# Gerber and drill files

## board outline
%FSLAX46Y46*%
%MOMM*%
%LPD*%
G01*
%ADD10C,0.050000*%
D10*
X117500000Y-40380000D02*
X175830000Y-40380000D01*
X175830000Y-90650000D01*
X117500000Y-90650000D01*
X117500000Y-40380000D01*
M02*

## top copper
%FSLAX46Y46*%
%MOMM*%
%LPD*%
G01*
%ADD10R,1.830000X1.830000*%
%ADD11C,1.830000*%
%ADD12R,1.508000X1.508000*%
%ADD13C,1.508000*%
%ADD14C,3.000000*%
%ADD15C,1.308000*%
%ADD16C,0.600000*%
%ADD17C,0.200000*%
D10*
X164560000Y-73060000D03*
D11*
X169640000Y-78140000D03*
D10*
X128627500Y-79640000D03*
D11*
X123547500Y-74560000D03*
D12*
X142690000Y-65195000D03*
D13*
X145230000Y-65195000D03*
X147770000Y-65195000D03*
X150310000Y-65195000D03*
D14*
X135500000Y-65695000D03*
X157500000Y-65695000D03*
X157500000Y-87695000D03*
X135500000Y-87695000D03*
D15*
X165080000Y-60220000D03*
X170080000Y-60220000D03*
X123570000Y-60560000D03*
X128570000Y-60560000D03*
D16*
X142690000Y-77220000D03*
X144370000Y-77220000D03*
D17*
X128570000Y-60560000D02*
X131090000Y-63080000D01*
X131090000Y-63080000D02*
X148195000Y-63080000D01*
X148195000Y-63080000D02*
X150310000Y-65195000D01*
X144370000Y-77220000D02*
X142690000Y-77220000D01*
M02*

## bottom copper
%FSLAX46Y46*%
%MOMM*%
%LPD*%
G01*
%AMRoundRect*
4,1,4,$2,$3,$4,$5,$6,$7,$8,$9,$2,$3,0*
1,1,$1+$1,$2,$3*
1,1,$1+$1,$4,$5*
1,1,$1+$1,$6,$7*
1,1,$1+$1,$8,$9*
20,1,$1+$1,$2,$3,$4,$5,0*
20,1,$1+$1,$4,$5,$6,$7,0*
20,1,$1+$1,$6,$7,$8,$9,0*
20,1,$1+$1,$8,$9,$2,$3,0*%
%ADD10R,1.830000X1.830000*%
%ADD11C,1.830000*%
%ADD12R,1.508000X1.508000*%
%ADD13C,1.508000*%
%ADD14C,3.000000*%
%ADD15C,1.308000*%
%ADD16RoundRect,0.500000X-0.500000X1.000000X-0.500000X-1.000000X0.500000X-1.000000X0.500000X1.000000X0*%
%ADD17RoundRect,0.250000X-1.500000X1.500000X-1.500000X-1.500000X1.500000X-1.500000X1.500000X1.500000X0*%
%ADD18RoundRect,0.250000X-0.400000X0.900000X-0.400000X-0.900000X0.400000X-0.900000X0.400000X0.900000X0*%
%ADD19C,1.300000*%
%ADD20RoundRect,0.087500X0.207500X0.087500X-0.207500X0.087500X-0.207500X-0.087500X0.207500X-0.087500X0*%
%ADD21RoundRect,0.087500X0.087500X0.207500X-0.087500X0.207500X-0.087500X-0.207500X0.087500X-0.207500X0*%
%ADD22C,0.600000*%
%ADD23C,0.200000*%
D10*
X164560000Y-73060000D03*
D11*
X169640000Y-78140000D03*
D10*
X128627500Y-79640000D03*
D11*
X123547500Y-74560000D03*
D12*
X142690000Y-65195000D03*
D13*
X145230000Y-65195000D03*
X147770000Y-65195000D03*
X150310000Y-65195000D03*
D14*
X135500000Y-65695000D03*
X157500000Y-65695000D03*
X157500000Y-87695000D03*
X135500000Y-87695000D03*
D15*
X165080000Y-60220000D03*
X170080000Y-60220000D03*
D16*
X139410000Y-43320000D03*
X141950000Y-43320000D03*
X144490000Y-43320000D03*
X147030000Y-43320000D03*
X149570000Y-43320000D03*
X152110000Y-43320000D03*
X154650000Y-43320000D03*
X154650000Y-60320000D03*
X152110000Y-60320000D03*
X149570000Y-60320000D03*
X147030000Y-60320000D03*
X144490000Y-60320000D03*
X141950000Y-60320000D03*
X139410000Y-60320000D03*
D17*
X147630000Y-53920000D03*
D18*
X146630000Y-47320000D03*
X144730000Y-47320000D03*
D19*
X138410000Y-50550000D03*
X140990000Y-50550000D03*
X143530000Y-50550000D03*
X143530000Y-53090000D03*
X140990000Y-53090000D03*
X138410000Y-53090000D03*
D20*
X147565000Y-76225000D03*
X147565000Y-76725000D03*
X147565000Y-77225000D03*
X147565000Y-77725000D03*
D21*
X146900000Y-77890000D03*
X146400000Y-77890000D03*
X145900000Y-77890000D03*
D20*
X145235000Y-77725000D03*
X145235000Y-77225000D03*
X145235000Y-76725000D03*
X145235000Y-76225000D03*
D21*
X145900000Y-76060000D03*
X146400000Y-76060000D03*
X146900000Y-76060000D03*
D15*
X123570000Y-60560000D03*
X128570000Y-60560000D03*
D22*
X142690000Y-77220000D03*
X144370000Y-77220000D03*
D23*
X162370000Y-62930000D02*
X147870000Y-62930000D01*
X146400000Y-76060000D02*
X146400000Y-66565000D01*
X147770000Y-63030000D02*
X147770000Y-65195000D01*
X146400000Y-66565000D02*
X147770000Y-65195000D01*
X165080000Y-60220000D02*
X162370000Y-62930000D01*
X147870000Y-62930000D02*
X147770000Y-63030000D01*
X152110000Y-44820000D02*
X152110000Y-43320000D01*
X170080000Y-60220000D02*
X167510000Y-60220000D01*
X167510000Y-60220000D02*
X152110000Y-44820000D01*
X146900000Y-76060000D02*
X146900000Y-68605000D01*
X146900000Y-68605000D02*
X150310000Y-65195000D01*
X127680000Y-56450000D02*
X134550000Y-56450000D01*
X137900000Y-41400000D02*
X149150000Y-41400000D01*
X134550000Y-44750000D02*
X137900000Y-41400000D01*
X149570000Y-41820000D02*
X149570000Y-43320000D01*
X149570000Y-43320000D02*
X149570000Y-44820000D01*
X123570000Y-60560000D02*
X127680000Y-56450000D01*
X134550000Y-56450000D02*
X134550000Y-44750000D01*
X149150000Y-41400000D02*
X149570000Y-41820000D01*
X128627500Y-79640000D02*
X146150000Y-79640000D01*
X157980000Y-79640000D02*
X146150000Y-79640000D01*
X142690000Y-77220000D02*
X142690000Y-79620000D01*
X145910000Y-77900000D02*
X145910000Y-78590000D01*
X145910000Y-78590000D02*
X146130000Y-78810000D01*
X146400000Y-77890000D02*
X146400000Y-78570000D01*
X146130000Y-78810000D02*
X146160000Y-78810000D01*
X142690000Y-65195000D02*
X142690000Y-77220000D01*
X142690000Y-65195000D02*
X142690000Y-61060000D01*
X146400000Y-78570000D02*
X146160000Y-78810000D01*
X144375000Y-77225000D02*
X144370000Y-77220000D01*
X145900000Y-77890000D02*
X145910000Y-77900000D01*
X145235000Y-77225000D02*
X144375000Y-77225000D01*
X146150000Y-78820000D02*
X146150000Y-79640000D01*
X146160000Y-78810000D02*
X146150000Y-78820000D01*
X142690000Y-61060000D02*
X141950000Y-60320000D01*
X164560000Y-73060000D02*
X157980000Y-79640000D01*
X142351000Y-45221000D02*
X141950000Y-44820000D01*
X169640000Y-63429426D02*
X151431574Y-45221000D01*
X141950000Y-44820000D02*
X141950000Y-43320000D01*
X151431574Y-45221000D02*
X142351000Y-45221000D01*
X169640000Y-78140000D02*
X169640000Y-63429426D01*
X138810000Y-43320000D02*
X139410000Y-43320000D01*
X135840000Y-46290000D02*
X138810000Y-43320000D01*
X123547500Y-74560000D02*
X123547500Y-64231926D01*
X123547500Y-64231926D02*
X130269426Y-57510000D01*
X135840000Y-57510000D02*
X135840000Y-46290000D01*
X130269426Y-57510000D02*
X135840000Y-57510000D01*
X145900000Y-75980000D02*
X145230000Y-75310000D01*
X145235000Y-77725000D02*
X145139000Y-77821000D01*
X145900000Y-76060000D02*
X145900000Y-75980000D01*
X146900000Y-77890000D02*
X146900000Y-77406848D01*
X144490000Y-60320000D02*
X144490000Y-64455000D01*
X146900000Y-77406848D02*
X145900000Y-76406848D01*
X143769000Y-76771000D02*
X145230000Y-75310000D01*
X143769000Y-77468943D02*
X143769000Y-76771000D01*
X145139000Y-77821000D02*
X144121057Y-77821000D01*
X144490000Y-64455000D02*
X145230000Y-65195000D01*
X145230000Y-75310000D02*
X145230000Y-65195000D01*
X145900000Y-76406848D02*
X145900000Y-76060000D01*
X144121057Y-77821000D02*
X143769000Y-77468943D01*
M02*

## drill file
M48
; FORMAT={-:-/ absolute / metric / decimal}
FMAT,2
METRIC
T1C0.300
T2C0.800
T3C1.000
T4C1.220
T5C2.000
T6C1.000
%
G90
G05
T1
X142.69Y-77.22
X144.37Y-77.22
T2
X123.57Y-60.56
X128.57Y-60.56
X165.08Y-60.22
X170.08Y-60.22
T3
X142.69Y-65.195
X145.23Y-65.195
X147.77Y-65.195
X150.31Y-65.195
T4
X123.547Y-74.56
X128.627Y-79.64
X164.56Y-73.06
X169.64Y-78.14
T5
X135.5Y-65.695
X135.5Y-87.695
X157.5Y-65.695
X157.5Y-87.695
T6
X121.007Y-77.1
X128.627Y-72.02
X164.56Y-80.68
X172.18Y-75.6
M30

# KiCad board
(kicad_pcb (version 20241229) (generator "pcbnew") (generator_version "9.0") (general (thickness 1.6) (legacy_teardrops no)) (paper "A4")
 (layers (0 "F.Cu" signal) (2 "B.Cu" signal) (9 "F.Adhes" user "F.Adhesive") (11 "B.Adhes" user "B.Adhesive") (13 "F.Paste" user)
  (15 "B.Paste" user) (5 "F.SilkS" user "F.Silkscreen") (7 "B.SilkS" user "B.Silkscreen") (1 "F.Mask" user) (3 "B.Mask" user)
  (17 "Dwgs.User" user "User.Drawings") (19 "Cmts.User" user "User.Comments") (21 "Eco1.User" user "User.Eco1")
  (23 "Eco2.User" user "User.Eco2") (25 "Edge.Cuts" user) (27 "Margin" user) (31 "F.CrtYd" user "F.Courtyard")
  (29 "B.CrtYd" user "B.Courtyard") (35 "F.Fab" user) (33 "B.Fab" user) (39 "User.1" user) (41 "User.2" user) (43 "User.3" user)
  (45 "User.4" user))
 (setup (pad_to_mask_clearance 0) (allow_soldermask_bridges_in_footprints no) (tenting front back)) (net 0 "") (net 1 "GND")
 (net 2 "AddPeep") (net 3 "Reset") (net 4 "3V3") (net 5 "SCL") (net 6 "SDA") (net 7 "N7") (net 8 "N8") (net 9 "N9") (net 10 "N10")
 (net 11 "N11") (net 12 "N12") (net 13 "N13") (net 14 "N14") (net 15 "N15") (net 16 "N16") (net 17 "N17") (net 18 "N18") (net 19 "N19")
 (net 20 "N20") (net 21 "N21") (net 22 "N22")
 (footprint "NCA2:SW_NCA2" (layer "F.Cu") (at 168.37 76.87 180)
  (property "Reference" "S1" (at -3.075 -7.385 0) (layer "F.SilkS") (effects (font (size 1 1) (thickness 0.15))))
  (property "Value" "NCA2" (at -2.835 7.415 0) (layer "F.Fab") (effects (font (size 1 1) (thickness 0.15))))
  (pad "" np_thru_hole circle (at -3.81 1.27 180) (size 1 1) (drill 1) (layers "*.Cu" "*.Mask"))
  (pad "" np_thru_hole circle (at 3.81 -3.81 180) (size 1 1) (drill 1) (layers "*.Cu" "*.Mask"))
  (pad "1" thru_hole rect (at 3.81 3.81 180) (size 1.83 1.83) (drill 1.22) (layers "*.Cu" "*.Mask") (remove_unused_layers no) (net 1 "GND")
   (solder_mask_margin 0.102))
  (pad "3" thru_hole circle (at -1.27 -1.27 180) (size 1.83 1.83) (drill 1.22) (layers "*.Cu" "*.Mask") (remove_unused_layers no)
   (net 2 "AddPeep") (solder_mask_margin 0.102)))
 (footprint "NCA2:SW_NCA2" (layer "F.Cu") (at 124.8175 75.83)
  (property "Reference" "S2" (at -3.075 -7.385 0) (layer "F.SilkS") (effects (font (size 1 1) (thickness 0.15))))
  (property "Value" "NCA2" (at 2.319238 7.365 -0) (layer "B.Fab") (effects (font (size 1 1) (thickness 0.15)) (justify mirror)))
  (pad "" np_thru_hole circle (at -3.81 1.27) (size 1 1) (drill 1) (layers "*.Cu" "*.Mask"))
  (pad "" np_thru_hole circle (at 3.81 -3.81) (size 1 1) (drill 1) (layers "*.Cu" "*.Mask"))
  (pad "1" thru_hole rect (at 3.81 3.81) (size 1.83 1.83) (drill 1.22) (layers "*.Cu" "*.Mask") (remove_unused_layers no) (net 1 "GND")
   (solder_mask_margin 0.102))
  (pad "3" thru_hole circle (at -1.27 -1.27) (size 1.83 1.83) (drill 1.22) (layers "*.Cu" "*.Mask") (remove_unused_layers no)
   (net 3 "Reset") (solder_mask_margin 0.102)))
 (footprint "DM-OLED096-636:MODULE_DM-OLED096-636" (layer "F.Cu") (at 146.5 76.695)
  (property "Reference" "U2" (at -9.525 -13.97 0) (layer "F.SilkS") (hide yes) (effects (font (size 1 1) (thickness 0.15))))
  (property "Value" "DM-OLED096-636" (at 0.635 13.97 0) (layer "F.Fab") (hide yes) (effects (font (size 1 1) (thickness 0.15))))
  (pad "1" thru_hole rect (at -3.81 -11.5) (size 1.508 1.508) (drill 1) (layers "*.Cu" "*.Mask") (remove_unused_layers no) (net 1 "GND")
   (solder_mask_margin 0.102))
  (pad "2" thru_hole circle (at -1.27 -11.5) (size 1.508 1.508) (drill 1) (layers "*.Cu" "*.Mask") (remove_unused_layers no) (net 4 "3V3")
   (solder_mask_margin 0.102))
  (pad "3" thru_hole circle (at 1.27 -11.5) (size 1.508 1.508) (drill 1) (layers "*.Cu" "*.Mask") (remove_unused_layers no) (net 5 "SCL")
   (solder_mask_margin 0.102))
  (pad "4" thru_hole circle (at 3.81 -11.5) (size 1.508 1.508) (drill 1) (layers "*.Cu" "*.Mask") (remove_unused_layers no) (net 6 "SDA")
   (solder_mask_margin 0.102))
  (pad "S1" thru_hole circle (at -11 -11) (size 3 3) (drill 2) (layers "*.Cu" "*.Mask") (remove_unused_layers no) (solder_mask_margin 0.102))
  (pad "S2" thru_hole circle (at 11 -11) (size 3 3) (drill 2) (layers "*.Cu" "*.Mask") (remove_unused_layers no) (solder_mask_margin 0.102))
  (pad "S3" thru_hole circle (at 11 11) (size 3 3) (drill 2) (layers "*.Cu" "*.Mask") (remove_unused_layers no) (solder_mask_margin 0.102))
  (pad "S4" thru_hole circle (at -11 11) (size 3 3) (drill 2) (layers "*.Cu" "*.Mask") (remove_unused_layers no) (solder_mask_margin 0.102)))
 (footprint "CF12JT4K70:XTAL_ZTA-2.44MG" (layer "B.Cu") (at 167.58 60.22)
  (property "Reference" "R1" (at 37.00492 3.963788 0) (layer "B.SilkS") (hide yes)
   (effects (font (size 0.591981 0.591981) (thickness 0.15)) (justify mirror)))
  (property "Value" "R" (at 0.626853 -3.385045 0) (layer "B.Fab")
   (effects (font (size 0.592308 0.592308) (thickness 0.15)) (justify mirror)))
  (pad "1" thru_hole circle (at -2.5 0) (size 1.308 1.308) (drill 0.8) (layers "*.Cu" "*.Mask") (remove_unused_layers no) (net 5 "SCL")
   (solder_mask_margin 0.102))
  (pad "2" thru_hole circle (at 2.5 0) (size 1.308 1.308) (drill 0.8) (layers "*.Cu" "*.Mask") (remove_unused_layers no) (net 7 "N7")
   (solder_mask_margin 0.102)))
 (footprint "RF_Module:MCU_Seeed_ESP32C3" (layer "B.Cu") (at 147.03 51.82 -90)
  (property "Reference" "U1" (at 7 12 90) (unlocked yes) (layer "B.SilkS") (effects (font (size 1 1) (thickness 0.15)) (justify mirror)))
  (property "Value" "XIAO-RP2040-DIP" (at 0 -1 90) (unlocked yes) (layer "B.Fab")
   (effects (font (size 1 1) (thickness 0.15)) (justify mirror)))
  (pad "" smd roundrect (at 1.1 -1.6 270) (size 1.5 1.5) (layers "B.Paste") (roundrect_rratio 0.1666666667))
  (pad "" smd roundrect (at 1.1 0.4 270) (size 1.5 1.5) (layers "B.Paste") (roundrect_rratio 0.1666666667))
  (pad "" smd roundrect (at 3.1 -1.6 270) (size 1.5 1.5) (layers "B.Paste") (roundrect_rratio 0.1666666667))
  (pad "" smd roundrect (at 3.1 0.4 270) (size 1.5 1.5) (layers "B.Paste") (roundrect_rratio 0.1666666667))
  (pad "1" smd roundrect (at -8.5 7.62 270) (size 3 2) (layers "B.Cu" "B.Mask" "B.Paste") (roundrect_rratio 0.25) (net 3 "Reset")
   (thermal_bridge_angle 45))
  (pad "2" smd roundrect (at -8.5 5.08 270) (size 3 2) (layers "B.Cu" "B.Mask" "B.Paste") (roundrect_rratio 0.25) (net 2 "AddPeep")
   (thermal_bridge_angle 45))
  (pad "3" smd roundrect (at -8.5 2.54 270) (size 3 2) (layers "B.Cu" "B.Mask" "B.Paste") (roundrect_rratio 0.25) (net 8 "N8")
   (thermal_bridge_angle 45))
  (pad "4" smd roundrect (at -8.5 0 270) (size 3 2) (layers "B.Cu" "B.Mask" "B.Paste") (roundrect_rratio 0.25) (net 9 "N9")
   (thermal_bridge_angle 45))
  (pad "5" smd roundrect (at -8.5 -2.54 270) (size 3 2) (layers "B.Cu" "B.Mask" "B.Paste") (roundrect_rratio 0.25) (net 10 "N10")
   (thermal_bridge_angle 45))
  (pad "6" smd roundrect (at -8.5 -5.08 270) (size 3 2) (layers "B.Cu" "B.Mask" "B.Paste") (roundrect_rratio 0.25) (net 7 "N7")
   (thermal_bridge_angle 45))
  (pad "7" smd roundrect (at -8.5 -7.62 270) (size 3 2) (layers "B.Cu" "B.Mask" "B.Paste") (roundrect_rratio 0.25) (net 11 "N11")
   (thermal_bridge_angle 45))
  (pad "8" smd roundrect (at 8.5 -7.62 270) (size 3 2) (layers "B.Cu" "B.Mask" "B.Paste") (roundrect_rratio 0.25) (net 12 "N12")
   (thermal_bridge_angle 45))
  (pad "9" smd roundrect (at 8.5 -5.08 270) (size 3 2) (layers "B.Cu" "B.Mask" "B.Paste") (roundrect_rratio 0.25) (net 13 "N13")
   (thermal_bridge_angle 45))
  (pad "10" smd roundrect (at 8.5 -2.54 270) (size 3 2) (layers "B.Cu" "B.Mask" "B.Paste") (roundrect_rratio 0.25) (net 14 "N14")
   (thermal_bridge_angle 45))
  (pad "11" smd roundrect (at 8.5 0 270) (size 3 2) (layers "B.Cu" "B.Mask" "B.Paste") (roundrect_rratio 0.25) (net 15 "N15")
   (thermal_bridge_angle 45))
  (pad "12" smd roundrect (at 8.5 2.54 270) (size 3 2) (layers "B.Cu" "B.Mask" "B.Paste") (roundrect_rratio 0.25) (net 4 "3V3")
   (thermal_bridge_angle 45))
  (pad "13" smd roundrect (at 8.5 5.08 270) (size 3 2) (layers "B.Cu" "B.Mask" "B.Paste") (roundrect_rratio 0.25) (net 1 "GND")
   (thermal_bridge_angle 45))
  (pad "14" smd roundrect (at 8.5 7.62 270) (size 3 2) (layers "B.Cu" "B.Mask" "B.Paste") (roundrect_rratio 0.25) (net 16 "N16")
   (thermal_bridge_angle 45))
  (pad "15" smd roundrect (at 2.1 -0.6 270) (size 3.5 3.5) (layers "B.Cu" "B.Mask") (roundrect_rratio 0.07142857143))
  (pad "16" smd roundrect (at -4.5 0.4 270) (size 2.3 1.3) (layers "B.Cu" "B.Mask" "B.Paste") (roundrect_rratio 0.1923076923))
  (pad "17" smd roundrect (at -4.5 2.3 270) (size 2.3 1.3) (layers "B.Cu" "B.Mask" "B.Paste") (roundrect_rratio 0.1923076923))
  (pad "18" smd circle (at -1.27 8.62 270) (size 1.3 1.3) (layers "B.Cu" "B.Mask" "B.Paste"))
  (pad "19" smd circle (at -1.27 6.04 270) (size 1.3 1.3) (layers "B.Cu" "B.Mask" "B.Paste"))
  (pad "20" smd circle (at -1.27 3.5 270) (size 1.3 1.3) (layers "B.Cu" "B.Mask" "B.Paste"))
  (pad "21" smd circle (at 1.27 3.5 270) (size 1.3 1.3) (layers "B.Cu" "B.Mask" "B.Paste"))
  (pad "22" smd circle (at 1.27 6.04 270) (size 1.3 1.3) (layers "B.Cu" "B.Mask" "B.Paste"))
  (pad "23" smd circle (at 1.27 8.62 270) (size 1.3 1.3) (layers "B.Cu" "B.Mask" "B.Paste")))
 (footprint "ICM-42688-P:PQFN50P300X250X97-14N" (layer "B.Cu") (at 146.4 76.975 180)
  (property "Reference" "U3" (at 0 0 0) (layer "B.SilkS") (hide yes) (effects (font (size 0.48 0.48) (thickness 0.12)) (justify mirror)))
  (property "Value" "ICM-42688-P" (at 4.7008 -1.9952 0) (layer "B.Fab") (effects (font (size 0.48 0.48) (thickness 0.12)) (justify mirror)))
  (pad "1" smd roundrect (at -1.165 0.75 180) (size 0.59 0.35) (layers "B.Cu" "B.Paste") (roundrect_rratio 0.25) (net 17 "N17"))
  (pad "2" smd roundrect (at -1.165 0.25 180) (size 0.59 0.35) (layers "B.Cu" "B.Paste") (roundrect_rratio 0.25) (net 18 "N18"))
  (pad "3" smd roundrect (at -1.165 -0.25 180) (size 0.59 0.35) (layers "B.Cu" "B.Paste") (roundrect_rratio 0.25) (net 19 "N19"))
  (pad "4" smd roundrect (at -1.165 -0.75 180) (size 0.59 0.35) (layers "B.Cu" "B.Paste") (roundrect_rratio 0.25) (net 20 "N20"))
  (pad "5" smd roundrect (at -0.5 -0.915 180) (size 0.35 0.59) (layers "B.Cu" "B.Paste") (roundrect_rratio 0.25) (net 4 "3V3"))
  (pad "6" smd roundrect (at 0 -0.915 180) (size 0.35 0.59) (layers "B.Cu" "B.Paste") (roundrect_rratio 0.25) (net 1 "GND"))
  (pad "7" smd roundrect (at 0.5 -0.915 180) (size 0.35 0.59) (layers "B.Cu" "B.Paste") (roundrect_rratio 0.25) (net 1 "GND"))
  (pad "8" smd roundrect (at 1.165 -0.75 180) (size 0.59 0.35) (layers "B.Cu" "B.Paste") (roundrect_rratio 0.25) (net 4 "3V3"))
  (pad "9" smd roundrect (at 1.165 -0.25 180) (size 0.59 0.35) (layers "B.Cu" "B.Paste") (roundrect_rratio 0.25) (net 1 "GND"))
  (pad "10" smd roundrect (at 1.165 0.25 180) (size 0.59 0.35) (layers "B.Cu" "B.Paste") (roundrect_rratio 0.25) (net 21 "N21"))
  (pad "11" smd roundrect (at 1.165 0.75 180) (size 0.59 0.35) (layers "B.Cu" "B.Paste") (roundrect_rratio 0.25) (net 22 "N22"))
  (pad "12" smd roundrect (at 0.5 0.915 180) (size 0.35 0.59) (layers "B.Cu" "B.Paste") (roundrect_rratio 0.25) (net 4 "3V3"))
  (pad "13" smd roundrect (at 0 0.915 180) (size 0.35 0.59) (layers "B.Cu" "B.Paste") (roundrect_rratio 0.25) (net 5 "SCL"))
  (pad "14" smd roundrect (at -0.5 0.915 180) (size 0.35 0.59) (layers "B.Cu" "B.Paste") (roundrect_rratio 0.25) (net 6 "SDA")))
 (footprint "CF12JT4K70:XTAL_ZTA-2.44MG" (layer "B.Cu") (at 126.07 60.56)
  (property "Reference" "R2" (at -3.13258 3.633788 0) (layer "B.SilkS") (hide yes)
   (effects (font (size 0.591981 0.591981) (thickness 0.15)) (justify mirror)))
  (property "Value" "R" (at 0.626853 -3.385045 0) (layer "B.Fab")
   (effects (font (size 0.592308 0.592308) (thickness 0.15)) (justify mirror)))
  (pad "1" thru_hole circle (at -2.5 0) (size 1.308 1.308) (drill 0.8) (layers "*.Cu" "*.Mask") (remove_unused_layers no) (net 10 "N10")
   (solder_mask_margin 0.102))
  (pad "2" thru_hole circle (at 2.5 0) (size 1.308 1.308) (drill 0.8) (layers "*.Cu" "*.Mask") (remove_unused_layers no) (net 6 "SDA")
   (solder_mask_margin 0.102)))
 (gr_rect (start 117.5 40.38) (end 175.83 90.65) (stroke (width 0.05) (type default)) (fill no) (layer "Edge.Cuts"))
 (segment (start 162.37 62.93) (end 147.87 62.93) (width 0.2) (layer "B.Cu") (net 5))
 (segment (start 146.4 76.06) (end 146.4 66.565) (width 0.2) (layer "B.Cu") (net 5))
 (segment (start 147.77 63.03) (end 147.77 65.195) (width 0.2) (layer "B.Cu") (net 5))
 (segment (start 146.4 66.565) (end 147.77 65.195) (width 0.2) (layer "B.Cu") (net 5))
 (segment (start 165.08 60.22) (end 162.37 62.93) (width 0.2) (layer "B.Cu") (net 5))
 (segment (start 147.87 62.93) (end 147.77 63.03) (width 0.2) (layer "B.Cu") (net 5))
 (segment (start 152.11 44.82) (end 152.11 43.32) (width 0.2) (layer "B.Cu") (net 7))
 (segment (start 170.08 60.22) (end 167.51 60.22) (width 0.2) (layer "B.Cu") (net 7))
 (segment (start 167.51 60.22) (end 152.11 44.82) (width 0.2) (layer "B.Cu") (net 7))
 (segment (start 128.57 60.56) (end 131.09 63.08) (width 0.2) (layer "F.Cu") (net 6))
 (segment (start 131.09 63.08) (end 148.195 63.08) (width 0.2) (layer "F.Cu") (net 6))
 (segment (start 148.195 63.08) (end 150.31 65.195) (width 0.2) (layer "F.Cu") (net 6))
 (segment (start 146.9 76.06) (end 146.9 68.605) (width 0.2) (layer "B.Cu") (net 6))
 (segment (start 146.9 68.605) (end 150.31 65.195) (width 0.2) (layer "B.Cu") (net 6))
 (segment (start 127.68 56.45) (end 134.55 56.45) (width 0.2) (layer "B.Cu") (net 10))
 (segment (start 137.9 41.4) (end 149.15 41.4) (width 0.2) (layer "B.Cu") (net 10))
 (segment (start 134.55 44.75) (end 137.9 41.4) (width 0.2) (layer "B.Cu") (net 10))
 (segment (start 149.57 41.82) (end 149.57 43.32) (width 0.2) (layer "B.Cu") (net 10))
 (segment (start 149.57 43.32) (end 149.57 44.82) (width 0.2) (layer "B.Cu") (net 10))
 (segment (start 123.57 60.56) (end 127.68 56.45) (width 0.2) (layer "B.Cu") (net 10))
 (segment (start 134.55 56.45) (end 134.55 44.75) (width 0.2) (layer "B.Cu") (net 10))
 (segment (start 149.15 41.4) (end 149.57 41.82) (width 0.2) (layer "B.Cu") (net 10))
 (segment (start 144.37 77.22) (end 142.69 77.22) (width 0.2) (layer "F.Cu") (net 1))
 (via (at 142.69 77.22) (size 0.6) (drill 0.3) (layers "F.Cu" "B.Cu") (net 1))
 (via (at 144.37 77.22) (size 0.6) (drill 0.3) (layers "F.Cu" "B.Cu") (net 1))
 (segment (start 128.6275 79.64) (end 146.15 79.64) (width 0.2) (layer "B.Cu") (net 1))
 (segment (start 157.98 79.64) (end 146.15 79.64) (width 0.2) (layer "B.Cu") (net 1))
 (segment (start 142.69 77.22) (end 142.69 79.62) (width 0.2) (layer "B.Cu") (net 1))
 (segment (start 145.91 77.9) (end 145.91 78.59) (width 0.2) (layer "B.Cu") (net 1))
 (segment (start 145.91 78.59) (end 146.13 78.81) (width 0.2) (layer "B.Cu") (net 1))
 (segment (start 146.4 77.89) (end 146.4 78.57) (width 0.2) (layer "B.Cu") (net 1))
 (segment (start 146.13 78.81) (end 146.16 78.81) (width 0.2) (layer "B.Cu") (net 1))
 (segment (start 142.69 65.195) (end 142.69 77.22) (width 0.2) (layer "B.Cu") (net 1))
 (segment (start 142.69 65.195) (end 142.69 61.06) (width 0.2) (layer "B.Cu") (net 1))
 (segment (start 146.4 78.57) (end 146.16 78.81) (width 0.2) (layer "B.Cu") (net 1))
 (segment (start 144.375 77.225) (end 144.37 77.22) (width 0.2) (layer "B.Cu") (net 1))
 (segment (start 145.9 77.89) (end 145.91 77.9) (width 0.2) (layer "B.Cu") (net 1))
 (segment (start 145.235 77.225) (end 144.375 77.225) (width 0.2) (layer "B.Cu") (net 1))
 (segment (start 146.15 78.82) (end 146.15 79.64) (width 0.2) (layer "B.Cu") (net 1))
 (segment (start 146.16 78.81) (end 146.15 78.82) (width 0.2) (layer "B.Cu") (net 1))
 (segment (start 142.69 61.06) (end 141.95 60.32) (width 0.2) (layer "B.Cu") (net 1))
 (segment (start 164.56 73.06) (end 157.98 79.64) (width 0.2) (layer "B.Cu") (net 1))
 (segment (start 142.351 45.221) (end 141.95 44.82) (width 0.2) (layer "B.Cu") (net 2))
 (segment (start 169.64 63.429426) (end 151.431574 45.221) (width 0.2) (layer "B.Cu") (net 2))
 (segment (start 141.95 44.82) (end 141.95 43.32) (width 0.2) (layer "B.Cu") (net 2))
 (segment (start 151.431574 45.221) (end 142.351 45.221) (width 0.2) (layer "B.Cu") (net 2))
 (segment (start 169.64 78.14) (end 169.64 63.429426) (width 0.2) (layer "B.Cu") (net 2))
 (segment (start 138.81 43.32) (end 139.41 43.32) (width 0.2) (layer "B.Cu") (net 3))
 (segment (start 135.84 46.29) (end 138.81 43.32) (width 0.2) (layer "B.Cu") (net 3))
 (segment (start 123.5475 74.56) (end 123.5475 64.231926) (width 0.2) (layer "B.Cu") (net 3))
 (segment (start 123.5475 64.231926) (end 130.269426 57.51) (width 0.2) (layer "B.Cu") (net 3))
 (segment (start 135.84 57.51) (end 135.84 46.29) (width 0.2) (layer "B.Cu") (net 3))
 (segment (start 130.269426 57.51) (end 135.84 57.51) (width 0.2) (layer "B.Cu") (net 3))
 (segment (start 145.9 75.98) (end 145.23 75.31) (width 0.2) (layer "B.Cu") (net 4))
 (segment (start 145.235 77.725) (end 145.139 77.821) (width 0.2) (layer "B.Cu") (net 4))
 (segment (start 145.9 76.06) (end 145.9 75.98) (width 0.2) (layer "B.Cu") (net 4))
 (segment (start 146.9 77.89) (end 146.9 77.406848) (width 0.2) (layer "B.Cu") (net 4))
 (segment (start 144.49 60.32) (end 144.49 64.455) (width 0.2) (layer "B.Cu") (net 4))
 (segment (start 146.9 77.406848) (end 145.9 76.406848) (width 0.2) (layer "B.Cu") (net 4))
 (segment (start 143.769 76.771) (end 145.23 75.31) (width 0.2) (layer "B.Cu") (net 4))
 (segment (start 143.769 77.468943) (end 143.769 76.771) (width 0.2) (layer "B.Cu") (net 4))
 (segment (start 145.139 77.821) (end 144.121057 77.821) (width 0.2) (layer "B.Cu") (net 4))
 (segment (start 144.49 64.455) (end 145.23 65.195) (width 0.2) (layer "B.Cu") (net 4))
 (segment (start 145.23 75.31) (end 145.23 65.195) (width 0.2) (layer "B.Cu") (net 4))
 (segment (start 145.9 76.406848) (end 145.9 76.06) (width 0.2) (layer "B.Cu") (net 4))
 (segment (start 144.121057 77.821) (end 143.769 77.468943) (width 0.2) (layer "B.Cu") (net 4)))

